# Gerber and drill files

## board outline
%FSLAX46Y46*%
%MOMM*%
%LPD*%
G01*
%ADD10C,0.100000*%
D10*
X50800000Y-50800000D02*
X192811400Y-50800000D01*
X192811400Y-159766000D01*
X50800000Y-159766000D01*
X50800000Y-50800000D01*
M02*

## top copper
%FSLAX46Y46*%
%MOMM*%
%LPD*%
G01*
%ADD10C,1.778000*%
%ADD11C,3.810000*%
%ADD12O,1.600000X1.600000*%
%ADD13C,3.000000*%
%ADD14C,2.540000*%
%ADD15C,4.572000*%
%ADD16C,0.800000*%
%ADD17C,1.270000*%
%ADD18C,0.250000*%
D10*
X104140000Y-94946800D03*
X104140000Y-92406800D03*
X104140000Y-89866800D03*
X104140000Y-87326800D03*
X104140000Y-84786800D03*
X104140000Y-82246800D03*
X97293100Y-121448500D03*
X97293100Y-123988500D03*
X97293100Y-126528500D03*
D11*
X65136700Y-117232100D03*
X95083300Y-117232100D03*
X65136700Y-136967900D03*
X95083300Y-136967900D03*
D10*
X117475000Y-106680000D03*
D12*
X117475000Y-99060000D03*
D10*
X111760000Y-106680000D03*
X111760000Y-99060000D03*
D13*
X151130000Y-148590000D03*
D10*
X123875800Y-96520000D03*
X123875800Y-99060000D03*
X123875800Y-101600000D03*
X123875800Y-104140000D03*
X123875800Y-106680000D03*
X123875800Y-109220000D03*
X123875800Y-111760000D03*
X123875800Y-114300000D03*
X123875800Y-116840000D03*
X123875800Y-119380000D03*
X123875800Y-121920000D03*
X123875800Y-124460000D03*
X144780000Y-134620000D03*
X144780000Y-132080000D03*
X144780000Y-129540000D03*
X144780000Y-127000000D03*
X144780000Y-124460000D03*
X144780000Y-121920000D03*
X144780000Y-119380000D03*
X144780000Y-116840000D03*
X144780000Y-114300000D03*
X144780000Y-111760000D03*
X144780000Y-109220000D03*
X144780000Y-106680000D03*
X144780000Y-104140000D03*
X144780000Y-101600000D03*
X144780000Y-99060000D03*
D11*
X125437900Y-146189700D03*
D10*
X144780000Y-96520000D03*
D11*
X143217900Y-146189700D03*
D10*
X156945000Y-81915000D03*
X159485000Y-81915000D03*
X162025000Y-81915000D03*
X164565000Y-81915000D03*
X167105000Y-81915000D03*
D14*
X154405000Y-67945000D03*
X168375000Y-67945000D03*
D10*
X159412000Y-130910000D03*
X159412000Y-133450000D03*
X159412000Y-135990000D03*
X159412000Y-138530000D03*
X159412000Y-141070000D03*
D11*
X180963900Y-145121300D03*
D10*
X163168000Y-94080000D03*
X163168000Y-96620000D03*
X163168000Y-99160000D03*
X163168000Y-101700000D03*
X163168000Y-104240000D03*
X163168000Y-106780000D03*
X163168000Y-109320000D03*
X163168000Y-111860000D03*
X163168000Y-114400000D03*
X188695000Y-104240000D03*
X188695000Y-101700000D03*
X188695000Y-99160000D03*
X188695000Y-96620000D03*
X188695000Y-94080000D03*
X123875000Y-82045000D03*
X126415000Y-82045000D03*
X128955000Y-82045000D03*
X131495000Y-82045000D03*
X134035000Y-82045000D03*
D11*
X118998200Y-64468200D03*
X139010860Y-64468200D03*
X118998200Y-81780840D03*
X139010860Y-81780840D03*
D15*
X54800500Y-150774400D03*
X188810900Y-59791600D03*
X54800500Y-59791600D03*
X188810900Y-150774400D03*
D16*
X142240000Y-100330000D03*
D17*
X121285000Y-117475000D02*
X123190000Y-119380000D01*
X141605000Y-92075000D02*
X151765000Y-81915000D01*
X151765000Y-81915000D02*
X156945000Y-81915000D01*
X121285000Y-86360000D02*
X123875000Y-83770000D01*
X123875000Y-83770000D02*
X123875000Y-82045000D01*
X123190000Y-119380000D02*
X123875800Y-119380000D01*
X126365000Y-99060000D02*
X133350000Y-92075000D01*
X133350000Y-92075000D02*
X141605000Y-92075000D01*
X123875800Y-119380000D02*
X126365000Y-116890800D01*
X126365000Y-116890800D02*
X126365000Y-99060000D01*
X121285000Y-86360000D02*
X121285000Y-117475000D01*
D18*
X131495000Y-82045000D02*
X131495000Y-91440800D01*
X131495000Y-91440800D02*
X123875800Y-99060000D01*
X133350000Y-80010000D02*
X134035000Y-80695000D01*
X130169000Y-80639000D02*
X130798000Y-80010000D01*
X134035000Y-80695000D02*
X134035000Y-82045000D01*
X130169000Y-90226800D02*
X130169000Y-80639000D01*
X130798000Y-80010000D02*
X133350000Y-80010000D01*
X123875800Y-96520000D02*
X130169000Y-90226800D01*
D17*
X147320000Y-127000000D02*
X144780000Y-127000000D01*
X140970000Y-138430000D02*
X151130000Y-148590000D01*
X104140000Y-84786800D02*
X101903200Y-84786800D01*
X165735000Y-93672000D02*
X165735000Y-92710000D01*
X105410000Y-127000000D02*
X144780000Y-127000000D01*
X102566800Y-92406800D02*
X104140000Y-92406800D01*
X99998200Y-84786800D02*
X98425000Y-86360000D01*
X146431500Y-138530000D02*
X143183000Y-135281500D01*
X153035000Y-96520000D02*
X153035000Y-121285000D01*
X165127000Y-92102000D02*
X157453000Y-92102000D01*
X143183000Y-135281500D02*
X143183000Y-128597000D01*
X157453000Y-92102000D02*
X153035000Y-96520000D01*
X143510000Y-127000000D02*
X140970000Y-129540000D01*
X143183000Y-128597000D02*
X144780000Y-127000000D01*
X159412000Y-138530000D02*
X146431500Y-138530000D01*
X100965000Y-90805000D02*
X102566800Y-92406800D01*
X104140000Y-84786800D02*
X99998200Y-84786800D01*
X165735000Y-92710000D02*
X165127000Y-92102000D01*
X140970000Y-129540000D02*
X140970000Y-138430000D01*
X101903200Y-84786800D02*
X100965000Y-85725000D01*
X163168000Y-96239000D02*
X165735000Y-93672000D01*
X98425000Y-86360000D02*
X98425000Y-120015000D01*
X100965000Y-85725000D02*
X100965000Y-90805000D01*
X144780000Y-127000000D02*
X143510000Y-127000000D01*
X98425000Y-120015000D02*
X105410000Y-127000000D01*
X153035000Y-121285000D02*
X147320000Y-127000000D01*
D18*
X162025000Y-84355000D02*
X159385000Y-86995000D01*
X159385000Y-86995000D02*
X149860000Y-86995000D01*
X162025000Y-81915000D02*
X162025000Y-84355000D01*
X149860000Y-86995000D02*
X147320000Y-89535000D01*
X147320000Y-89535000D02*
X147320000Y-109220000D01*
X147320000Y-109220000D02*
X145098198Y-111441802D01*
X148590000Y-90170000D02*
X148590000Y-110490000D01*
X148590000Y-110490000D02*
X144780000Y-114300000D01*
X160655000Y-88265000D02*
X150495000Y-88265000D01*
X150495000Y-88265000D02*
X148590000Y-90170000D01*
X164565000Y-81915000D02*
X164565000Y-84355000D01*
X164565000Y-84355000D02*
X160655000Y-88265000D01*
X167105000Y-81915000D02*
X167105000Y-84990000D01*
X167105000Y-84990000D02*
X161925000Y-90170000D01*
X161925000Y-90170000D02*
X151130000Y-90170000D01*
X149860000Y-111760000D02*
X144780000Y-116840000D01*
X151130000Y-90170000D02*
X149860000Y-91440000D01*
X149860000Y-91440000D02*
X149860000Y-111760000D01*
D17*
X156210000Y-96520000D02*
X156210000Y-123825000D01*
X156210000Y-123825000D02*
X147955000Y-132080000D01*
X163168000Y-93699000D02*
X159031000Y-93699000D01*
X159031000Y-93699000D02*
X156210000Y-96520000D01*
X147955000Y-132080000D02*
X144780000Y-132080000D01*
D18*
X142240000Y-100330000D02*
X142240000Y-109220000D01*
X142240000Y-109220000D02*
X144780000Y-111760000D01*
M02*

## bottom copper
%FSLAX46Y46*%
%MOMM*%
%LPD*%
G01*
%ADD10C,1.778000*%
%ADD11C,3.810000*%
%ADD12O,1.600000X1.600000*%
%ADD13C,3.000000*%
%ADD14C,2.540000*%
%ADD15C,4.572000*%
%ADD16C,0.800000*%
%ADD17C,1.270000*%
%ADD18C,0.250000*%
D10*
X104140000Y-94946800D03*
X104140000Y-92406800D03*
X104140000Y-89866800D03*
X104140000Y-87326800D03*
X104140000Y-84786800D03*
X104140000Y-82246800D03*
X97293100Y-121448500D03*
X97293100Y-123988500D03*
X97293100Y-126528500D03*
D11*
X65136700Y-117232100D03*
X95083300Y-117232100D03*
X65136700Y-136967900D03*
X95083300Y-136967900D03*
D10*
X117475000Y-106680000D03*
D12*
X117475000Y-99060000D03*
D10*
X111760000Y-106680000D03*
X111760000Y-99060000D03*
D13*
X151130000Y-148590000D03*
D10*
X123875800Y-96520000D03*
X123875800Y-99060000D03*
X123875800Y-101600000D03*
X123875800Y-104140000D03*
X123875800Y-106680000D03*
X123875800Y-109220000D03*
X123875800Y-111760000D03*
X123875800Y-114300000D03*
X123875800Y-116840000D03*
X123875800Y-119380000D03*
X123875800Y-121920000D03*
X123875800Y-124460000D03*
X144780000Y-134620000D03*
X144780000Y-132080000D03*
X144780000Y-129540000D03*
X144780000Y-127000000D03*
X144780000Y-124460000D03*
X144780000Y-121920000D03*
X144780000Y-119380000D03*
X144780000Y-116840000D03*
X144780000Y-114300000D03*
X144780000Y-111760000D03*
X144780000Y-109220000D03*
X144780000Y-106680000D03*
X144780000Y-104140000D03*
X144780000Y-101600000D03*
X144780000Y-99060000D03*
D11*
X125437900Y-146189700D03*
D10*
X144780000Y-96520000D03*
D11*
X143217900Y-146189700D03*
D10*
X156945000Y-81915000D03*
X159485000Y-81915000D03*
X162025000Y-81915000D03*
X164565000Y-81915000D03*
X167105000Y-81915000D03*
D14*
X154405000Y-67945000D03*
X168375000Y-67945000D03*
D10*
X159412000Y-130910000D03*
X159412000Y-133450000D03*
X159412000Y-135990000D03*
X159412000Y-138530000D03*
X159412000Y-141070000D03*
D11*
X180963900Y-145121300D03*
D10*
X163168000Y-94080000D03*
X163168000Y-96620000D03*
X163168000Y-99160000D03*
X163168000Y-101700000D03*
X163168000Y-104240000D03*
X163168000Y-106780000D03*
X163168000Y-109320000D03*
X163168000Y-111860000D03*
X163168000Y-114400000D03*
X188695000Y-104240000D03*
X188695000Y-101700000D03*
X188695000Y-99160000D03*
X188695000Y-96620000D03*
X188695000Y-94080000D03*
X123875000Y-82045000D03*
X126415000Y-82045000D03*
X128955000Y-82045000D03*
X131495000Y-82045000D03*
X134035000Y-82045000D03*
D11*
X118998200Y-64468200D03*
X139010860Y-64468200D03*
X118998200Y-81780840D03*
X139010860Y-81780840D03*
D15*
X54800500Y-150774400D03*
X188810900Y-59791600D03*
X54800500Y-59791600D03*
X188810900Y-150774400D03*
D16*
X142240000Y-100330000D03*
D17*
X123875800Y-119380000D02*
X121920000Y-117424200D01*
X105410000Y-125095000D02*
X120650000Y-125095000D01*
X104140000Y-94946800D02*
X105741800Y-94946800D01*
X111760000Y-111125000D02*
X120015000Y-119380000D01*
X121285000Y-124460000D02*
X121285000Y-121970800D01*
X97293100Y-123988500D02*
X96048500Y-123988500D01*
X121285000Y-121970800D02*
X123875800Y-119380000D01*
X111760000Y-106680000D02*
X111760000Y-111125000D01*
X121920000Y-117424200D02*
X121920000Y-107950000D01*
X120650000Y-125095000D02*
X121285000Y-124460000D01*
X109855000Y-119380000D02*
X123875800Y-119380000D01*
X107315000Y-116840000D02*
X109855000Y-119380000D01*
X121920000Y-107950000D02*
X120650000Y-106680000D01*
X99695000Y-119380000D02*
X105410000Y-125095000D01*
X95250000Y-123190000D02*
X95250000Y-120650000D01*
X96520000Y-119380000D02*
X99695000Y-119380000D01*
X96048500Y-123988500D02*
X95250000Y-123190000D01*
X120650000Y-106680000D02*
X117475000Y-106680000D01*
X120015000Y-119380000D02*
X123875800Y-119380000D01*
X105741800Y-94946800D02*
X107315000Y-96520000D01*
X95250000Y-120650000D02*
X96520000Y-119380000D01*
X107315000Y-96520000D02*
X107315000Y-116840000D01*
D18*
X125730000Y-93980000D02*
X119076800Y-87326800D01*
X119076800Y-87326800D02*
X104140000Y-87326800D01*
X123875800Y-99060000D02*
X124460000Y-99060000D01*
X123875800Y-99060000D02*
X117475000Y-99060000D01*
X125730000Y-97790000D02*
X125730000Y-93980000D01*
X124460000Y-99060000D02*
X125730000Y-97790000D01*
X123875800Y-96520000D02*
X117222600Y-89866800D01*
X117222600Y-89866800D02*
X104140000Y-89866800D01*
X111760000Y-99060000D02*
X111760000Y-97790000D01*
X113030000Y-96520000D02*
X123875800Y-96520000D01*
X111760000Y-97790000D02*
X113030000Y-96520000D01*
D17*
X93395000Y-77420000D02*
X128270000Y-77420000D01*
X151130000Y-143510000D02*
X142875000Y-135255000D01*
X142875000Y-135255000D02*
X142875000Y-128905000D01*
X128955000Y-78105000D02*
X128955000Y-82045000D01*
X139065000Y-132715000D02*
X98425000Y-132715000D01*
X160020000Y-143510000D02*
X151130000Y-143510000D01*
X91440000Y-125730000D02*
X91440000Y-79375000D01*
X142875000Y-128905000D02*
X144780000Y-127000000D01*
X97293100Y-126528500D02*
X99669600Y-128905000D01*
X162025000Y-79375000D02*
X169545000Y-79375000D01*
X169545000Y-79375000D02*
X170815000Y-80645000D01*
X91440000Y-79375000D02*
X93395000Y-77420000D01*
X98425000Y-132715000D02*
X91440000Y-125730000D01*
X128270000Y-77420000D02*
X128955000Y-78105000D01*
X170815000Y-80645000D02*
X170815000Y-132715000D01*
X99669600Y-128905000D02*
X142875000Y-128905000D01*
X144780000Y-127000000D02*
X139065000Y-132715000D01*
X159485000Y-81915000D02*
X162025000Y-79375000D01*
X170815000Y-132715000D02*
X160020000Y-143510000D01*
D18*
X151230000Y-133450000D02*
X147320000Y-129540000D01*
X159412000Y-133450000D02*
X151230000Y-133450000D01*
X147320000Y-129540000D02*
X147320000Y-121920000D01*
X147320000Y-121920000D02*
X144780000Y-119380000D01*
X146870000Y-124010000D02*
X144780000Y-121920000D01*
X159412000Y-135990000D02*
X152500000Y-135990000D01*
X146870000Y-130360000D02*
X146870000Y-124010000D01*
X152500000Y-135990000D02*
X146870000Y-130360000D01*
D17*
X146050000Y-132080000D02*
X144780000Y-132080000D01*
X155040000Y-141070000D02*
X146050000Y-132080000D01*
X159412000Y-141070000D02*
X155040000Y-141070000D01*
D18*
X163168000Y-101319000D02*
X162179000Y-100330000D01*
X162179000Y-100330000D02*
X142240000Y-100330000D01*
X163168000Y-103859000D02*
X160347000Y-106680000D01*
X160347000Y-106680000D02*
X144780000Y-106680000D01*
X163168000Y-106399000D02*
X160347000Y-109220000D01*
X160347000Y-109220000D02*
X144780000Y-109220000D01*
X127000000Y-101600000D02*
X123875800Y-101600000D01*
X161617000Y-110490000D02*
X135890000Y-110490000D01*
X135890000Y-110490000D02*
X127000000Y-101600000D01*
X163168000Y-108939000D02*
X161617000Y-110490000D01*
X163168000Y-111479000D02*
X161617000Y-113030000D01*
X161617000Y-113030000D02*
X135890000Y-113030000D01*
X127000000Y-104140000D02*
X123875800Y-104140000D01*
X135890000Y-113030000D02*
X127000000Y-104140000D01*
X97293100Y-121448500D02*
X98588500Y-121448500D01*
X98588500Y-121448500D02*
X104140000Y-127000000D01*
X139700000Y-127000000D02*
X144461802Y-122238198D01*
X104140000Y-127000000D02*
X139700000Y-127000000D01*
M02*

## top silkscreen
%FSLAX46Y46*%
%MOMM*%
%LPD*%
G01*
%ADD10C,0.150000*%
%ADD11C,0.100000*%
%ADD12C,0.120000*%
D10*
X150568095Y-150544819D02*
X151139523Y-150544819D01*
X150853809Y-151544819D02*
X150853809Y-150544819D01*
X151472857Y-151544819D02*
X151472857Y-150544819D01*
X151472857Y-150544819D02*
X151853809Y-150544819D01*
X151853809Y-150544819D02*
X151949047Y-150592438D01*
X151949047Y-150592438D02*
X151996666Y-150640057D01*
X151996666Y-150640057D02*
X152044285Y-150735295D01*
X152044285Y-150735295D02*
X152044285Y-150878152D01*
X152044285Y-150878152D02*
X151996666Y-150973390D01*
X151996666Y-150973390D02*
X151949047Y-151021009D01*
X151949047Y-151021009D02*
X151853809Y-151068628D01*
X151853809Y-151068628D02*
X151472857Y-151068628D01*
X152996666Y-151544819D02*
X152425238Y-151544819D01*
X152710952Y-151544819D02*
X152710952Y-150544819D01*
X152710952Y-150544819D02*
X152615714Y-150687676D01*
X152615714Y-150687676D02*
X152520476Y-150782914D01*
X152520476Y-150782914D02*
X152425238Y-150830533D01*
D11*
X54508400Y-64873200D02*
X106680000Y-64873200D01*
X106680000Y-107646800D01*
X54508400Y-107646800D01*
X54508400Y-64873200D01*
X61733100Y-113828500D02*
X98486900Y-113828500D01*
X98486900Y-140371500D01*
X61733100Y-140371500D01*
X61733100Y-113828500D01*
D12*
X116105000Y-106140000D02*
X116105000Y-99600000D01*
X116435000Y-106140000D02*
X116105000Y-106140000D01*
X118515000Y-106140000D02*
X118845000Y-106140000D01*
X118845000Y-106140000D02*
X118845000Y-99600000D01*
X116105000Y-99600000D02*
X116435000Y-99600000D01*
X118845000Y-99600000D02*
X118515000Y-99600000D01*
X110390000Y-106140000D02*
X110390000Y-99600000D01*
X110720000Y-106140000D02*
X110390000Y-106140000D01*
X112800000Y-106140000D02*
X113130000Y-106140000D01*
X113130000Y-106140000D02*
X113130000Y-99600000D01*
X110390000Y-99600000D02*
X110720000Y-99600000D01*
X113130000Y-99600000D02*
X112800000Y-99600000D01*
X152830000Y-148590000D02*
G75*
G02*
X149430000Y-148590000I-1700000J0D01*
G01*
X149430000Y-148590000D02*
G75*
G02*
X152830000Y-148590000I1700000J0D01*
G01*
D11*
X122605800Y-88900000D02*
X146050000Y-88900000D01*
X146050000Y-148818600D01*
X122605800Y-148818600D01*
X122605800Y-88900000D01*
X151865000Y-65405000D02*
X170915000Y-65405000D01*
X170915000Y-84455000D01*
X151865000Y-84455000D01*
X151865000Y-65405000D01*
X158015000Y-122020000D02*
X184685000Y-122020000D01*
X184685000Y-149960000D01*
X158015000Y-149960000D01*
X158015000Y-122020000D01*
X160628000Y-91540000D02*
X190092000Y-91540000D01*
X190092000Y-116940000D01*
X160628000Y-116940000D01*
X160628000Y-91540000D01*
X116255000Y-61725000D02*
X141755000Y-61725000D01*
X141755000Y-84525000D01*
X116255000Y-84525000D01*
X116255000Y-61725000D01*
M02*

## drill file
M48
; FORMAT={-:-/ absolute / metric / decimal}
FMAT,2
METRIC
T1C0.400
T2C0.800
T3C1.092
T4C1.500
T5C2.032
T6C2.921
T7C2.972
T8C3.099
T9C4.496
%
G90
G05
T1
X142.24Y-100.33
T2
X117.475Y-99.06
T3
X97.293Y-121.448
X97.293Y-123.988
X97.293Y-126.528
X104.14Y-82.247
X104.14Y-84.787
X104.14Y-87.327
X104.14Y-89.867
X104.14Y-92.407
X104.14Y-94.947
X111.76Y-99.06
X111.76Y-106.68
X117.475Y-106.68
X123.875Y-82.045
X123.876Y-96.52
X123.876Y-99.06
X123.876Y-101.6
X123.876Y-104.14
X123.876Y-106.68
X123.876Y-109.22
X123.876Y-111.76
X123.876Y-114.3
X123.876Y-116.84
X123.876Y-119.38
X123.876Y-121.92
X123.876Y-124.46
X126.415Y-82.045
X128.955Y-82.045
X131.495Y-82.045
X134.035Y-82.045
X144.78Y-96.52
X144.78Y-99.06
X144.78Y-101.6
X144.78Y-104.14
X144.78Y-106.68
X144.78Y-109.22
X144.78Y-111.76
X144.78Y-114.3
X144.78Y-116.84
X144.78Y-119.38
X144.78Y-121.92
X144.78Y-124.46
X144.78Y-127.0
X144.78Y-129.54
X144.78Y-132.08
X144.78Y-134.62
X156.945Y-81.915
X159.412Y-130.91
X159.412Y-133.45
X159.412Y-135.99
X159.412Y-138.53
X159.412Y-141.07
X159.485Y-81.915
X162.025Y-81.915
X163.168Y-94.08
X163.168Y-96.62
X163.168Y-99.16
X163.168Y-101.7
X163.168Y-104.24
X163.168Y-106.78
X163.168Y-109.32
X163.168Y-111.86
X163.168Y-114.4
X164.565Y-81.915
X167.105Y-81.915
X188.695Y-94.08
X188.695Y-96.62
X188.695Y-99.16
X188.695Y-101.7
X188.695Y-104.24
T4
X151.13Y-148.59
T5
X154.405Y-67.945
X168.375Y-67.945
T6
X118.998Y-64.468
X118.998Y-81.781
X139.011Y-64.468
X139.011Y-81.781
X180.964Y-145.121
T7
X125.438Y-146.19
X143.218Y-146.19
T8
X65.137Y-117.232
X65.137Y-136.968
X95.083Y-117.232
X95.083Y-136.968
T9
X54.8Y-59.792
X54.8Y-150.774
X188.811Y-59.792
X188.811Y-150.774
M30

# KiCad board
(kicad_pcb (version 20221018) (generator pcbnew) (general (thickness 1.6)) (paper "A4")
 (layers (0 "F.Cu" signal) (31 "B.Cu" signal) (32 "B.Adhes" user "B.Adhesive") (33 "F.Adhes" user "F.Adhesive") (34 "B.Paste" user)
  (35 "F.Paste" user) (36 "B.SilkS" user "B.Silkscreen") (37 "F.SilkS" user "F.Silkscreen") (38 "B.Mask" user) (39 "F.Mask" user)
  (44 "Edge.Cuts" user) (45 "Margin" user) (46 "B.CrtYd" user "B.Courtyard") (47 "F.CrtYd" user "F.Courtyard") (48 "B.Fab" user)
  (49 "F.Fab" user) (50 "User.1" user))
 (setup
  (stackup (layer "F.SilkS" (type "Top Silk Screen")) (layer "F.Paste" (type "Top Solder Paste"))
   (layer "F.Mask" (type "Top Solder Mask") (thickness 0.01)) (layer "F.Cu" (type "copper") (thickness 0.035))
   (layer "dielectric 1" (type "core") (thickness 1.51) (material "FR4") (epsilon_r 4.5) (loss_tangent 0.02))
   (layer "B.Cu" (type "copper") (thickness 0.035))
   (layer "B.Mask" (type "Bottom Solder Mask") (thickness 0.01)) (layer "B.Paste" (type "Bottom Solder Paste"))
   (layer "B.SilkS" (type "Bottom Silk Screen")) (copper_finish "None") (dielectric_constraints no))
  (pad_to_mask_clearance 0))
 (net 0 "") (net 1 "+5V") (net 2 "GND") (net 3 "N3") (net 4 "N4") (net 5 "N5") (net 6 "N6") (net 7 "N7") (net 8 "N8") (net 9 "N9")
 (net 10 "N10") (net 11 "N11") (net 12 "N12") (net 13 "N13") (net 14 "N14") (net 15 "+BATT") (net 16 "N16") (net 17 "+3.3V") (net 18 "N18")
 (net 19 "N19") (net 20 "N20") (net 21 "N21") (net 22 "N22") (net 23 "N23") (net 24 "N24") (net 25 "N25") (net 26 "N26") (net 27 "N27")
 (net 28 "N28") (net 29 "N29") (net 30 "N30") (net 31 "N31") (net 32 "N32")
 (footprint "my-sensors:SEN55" (layer "F.Cu") (at 106.68 107.6468 180)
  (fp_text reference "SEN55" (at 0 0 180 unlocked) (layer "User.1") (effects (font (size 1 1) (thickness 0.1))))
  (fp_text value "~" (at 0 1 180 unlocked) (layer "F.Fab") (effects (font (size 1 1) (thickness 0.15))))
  (fp_rect (start 0 0) (end 52.1716 42.7736) (stroke (width 0.1) (type default)) (fill none) (layer "F.SilkS"))
  (pad "1" thru_hole circle (at 2.54 12.7 180) (size 1.778 1.778) (drill 1.0922) (layers "*.Cu" "*.Mask") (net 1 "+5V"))
  (pad "2" thru_hole circle (at 2.54 15.24 180) (size 1.778 1.778) (drill 1.0922) (layers "*.Cu" "*.Mask") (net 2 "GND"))
  (pad "3" thru_hole circle (at 2.54 17.78 180) (size 1.778 1.778) (drill 1.0922) (layers "*.Cu" "*.Mask") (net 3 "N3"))
  (pad "4" thru_hole circle (at 2.54 20.32 180) (size 1.778 1.778) (drill 1.0922) (layers "*.Cu" "*.Mask") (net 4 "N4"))
  (pad "5" thru_hole circle (at 2.54 22.86 180) (size 1.778 1.778) (drill 1.0922) (layers "*.Cu" "*.Mask") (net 2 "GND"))
  (pad "6" thru_hole circle (at 2.54 25.4 180) (size 1.778 1.778) (drill 1.0922) (layers "*.Cu" "*.Mask") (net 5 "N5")))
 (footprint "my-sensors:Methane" (layer "F.Cu") (at 61.7331 113.8285)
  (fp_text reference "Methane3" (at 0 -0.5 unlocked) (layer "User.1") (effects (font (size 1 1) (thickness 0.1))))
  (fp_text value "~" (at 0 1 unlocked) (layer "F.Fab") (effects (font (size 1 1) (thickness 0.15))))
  (fp_rect (start 0 0) (end 36.7538 26.543) (stroke (width 0.1) (type default)) (fill none) (layer "F.SilkS"))
  (pad "1" thru_hole circle (at 35.56 7.62) (size 1.778 1.778) (drill 1.0922) (layers "*.Cu" "*.Mask") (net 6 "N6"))
  (pad "2" thru_hole circle (at 35.56 10.16) (size 1.778 1.778) (drill 1.0922) (layers "*.Cu" "*.Mask") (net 1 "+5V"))
  (pad "3" thru_hole circle (at 35.56 12.7) (size 1.778 1.778) (drill 1.0922) (layers "*.Cu" "*.Mask") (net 2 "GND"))
  (pad "4" thru_hole circle (at 3.4036 3.4036 270) (size 3.81 3.81) (drill 3.0988) (layers "*.Cu" "*.Mask"))
  (pad "5" thru_hole circle (at 33.3502 3.4036 270) (size 3.81 3.81) (drill 3.0988) (layers "*.Cu" "*.Mask"))
  (pad "6" thru_hole circle (at 3.4036 23.1394 270) (size 3.81 3.81) (drill 3.0988) (layers "*.Cu" "*.Mask"))
  (pad "7" thru_hole circle (at 33.3502 23.1394 270) (size 3.81 3.81) (drill 3.0988) (layers "*.Cu" "*.Mask")))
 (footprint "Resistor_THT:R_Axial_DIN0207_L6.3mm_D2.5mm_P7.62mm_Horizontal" (layer "F.Cu") (at 117.475 106.68 90)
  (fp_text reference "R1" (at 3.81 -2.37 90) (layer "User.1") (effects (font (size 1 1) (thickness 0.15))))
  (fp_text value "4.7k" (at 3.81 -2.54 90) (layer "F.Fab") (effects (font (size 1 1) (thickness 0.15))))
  (fp_line (start 0.54 -1.37) (end 7.08 -1.37) (stroke (width 0.12) (type solid)) (layer "F.SilkS"))
  (fp_line (start 0.54 -1.04) (end 0.54 -1.37) (stroke (width 0.12) (type solid)) (layer "F.SilkS"))
  (fp_line (start 0.54 1.04) (end 0.54 1.37) (stroke (width 0.12) (type solid)) (layer "F.SilkS"))
  (fp_line (start 0.54 1.37) (end 7.08 1.37) (stroke (width 0.12) (type solid)) (layer "F.SilkS"))
  (fp_line (start 7.08 -1.37) (end 7.08 -1.04) (stroke (width 0.12) (type solid)) (layer "F.SilkS"))
  (fp_line (start 7.08 1.37) (end 7.08 1.04) (stroke (width 0.12) (type solid)) (layer "F.SilkS"))
  (pad "1" thru_hole circle (at 0 0 90) (size 1.778 1.778) (drill 1.0922) (layers "*.Cu" "*.Mask") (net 1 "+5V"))
  (pad "2" thru_hole oval (at 7.62 0 90) (size 1.6 1.6) (drill 0.8) (layers "*.Cu" "*.Mask") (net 4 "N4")))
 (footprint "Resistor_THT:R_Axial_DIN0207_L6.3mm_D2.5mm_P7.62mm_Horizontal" (layer "F.Cu") (at 111.76 106.68 90)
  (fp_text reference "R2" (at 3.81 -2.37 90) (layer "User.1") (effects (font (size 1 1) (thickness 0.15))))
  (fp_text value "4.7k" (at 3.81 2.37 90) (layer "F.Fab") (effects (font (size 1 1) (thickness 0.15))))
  (fp_line (start 0.54 -1.37) (end 7.08 -1.37) (stroke (width 0.12) (type solid)) (layer "F.SilkS"))
  (fp_line (start 0.54 -1.04) (end 0.54 -1.37) (stroke (width 0.12) (type solid)) (layer "F.SilkS"))
  (fp_line (start 0.54 1.04) (end 0.54 1.37) (stroke (width 0.12) (type solid)) (layer "F.SilkS"))
  (fp_line (start 0.54 1.37) (end 7.08 1.37) (stroke (width 0.12) (type solid)) (layer "F.SilkS"))
  (fp_line (start 7.08 -1.37) (end 7.08 -1.04) (stroke (width 0.12) (type solid)) (layer "F.SilkS"))
  (fp_line (start 7.08 1.37) (end 7.08 1.04) (stroke (width 0.12) (type solid)) (layer "F.SilkS"))
  (pad "1" thru_hole circle (at 0 0 90) (size 1.778 1.778) (drill 1.0922) (layers "*.Cu" "*.Mask") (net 1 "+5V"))
  (pad "2" thru_hole circle (at 7.62 0 90) (size 1.778 1.778) (drill 1.0922) (layers "*.Cu" "*.Mask") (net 3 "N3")))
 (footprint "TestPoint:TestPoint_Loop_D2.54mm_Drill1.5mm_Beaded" (layer "F.Cu") (at 151.13 148.59)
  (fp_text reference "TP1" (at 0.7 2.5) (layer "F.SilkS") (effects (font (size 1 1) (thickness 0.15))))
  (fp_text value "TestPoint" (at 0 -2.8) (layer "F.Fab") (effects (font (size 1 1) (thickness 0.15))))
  (fp_circle (center 0 0) (end 1.7 0) (stroke (width 0.12) (type solid)) (fill none) (layer "F.SilkS"))
  (pad "1" thru_hole circle (at 0 0) (size 3 3) (drill 1.5) (layers "*.Cu" "*.Mask") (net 2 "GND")))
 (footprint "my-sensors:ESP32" (layer "F.Cu") (at 122.6058 88.9)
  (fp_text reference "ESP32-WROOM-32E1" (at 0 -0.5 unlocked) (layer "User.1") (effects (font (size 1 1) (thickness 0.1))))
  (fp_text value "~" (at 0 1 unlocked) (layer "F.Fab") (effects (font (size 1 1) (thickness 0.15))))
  (fp_rect (start 0 0) (end 23.4442 59.9186) (stroke (width 0.1) (type default)) (fill none) (layer "F.SilkS"))
  (pad "1" thru_hole circle (at 1.27 7.62) (size 1.778 1.778) (drill 1.0922) (layers "*.Cu" "*.Mask") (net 3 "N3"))
  (pad "2" thru_hole circle (at 1.27 10.16) (size 1.778 1.778) (drill 1.0922) (layers "*.Cu" "*.Mask") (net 4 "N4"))
  (pad "3" thru_hole circle (at 1.27 12.7) (size 1.778 1.778) (drill 1.0922) (layers "*.Cu" "*.Mask") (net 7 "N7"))
  (pad "4" thru_hole circle (at 1.27 15.24) (size 1.778 1.778) (drill 1.0922) (layers "*.Cu" "*.Mask") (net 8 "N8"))
  (pad "5" thru_hole circle (at 1.27 17.78) (size 1.778 1.778) (drill 1.0922) (layers "*.Cu" "*.Mask") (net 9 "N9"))
  (pad "6" thru_hole circle (at 1.27 20.32) (size 1.778 1.778) (drill 1.0922) (layers "*.Cu" "*.Mask") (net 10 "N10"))
  (pad "7" thru_hole circle (at 1.27 22.86) (size 1.778 1.778) (drill 1.0922) (layers "*.Cu" "*.Mask") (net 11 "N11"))
  (pad "8" thru_hole circle (at 1.27 25.4) (size 1.778 1.778) (drill 1.0922) (layers "*.Cu" "*.Mask") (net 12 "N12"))
  (pad "9" thru_hole circle (at 1.27 27.94) (size 1.778 1.778) (drill 1.0922) (layers "*.Cu" "*.Mask") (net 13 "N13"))
  (pad "10" thru_hole circle (at 1.27 30.48) (size 1.778 1.778) (drill 1.0922) (layers "*.Cu" "*.Mask") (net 1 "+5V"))
  (pad "11" thru_hole circle (at 1.27 33.02) (size 1.778 1.778) (drill 1.0922) (layers "*.Cu" "*.Mask") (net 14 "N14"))
  (pad "12" thru_hole circle (at 1.27 35.56) (size 1.778 1.778) (drill 1.0922) (layers "*.Cu" "*.Mask") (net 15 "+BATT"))
  (pad "13" thru_hole circle (at 22.1742 45.72) (size 1.778 1.778) (drill 1.0922) (layers "*.Cu" "*.Mask") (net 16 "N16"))
  (pad "14" thru_hole circle (at 22.1742 43.18) (size 1.778 1.778) (drill 1.0922) (layers "*.Cu" "*.Mask") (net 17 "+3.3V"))
  (pad "15" thru_hole circle (at 22.1742 40.64) (size 1.778 1.778) (drill 1.0922) (layers "*.Cu" "*.Mask") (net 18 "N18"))
  (pad "16" thru_hole circle (at 22.1742 38.1) (size 1.778 1.778) (drill 1.0922) (layers "*.Cu" "*.Mask") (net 2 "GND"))
  (pad "17" thru_hole circle (at 22.1742 35.56) (size 1.778 1.778) (drill 1.0922) (layers "*.Cu" "*.Mask") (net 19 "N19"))
  (pad "18" thru_hole circle (at 22.1742 33.02) (size 1.778 1.778) (drill 1.0922) (layers "*.Cu" "*.Mask") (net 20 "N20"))
  (pad "19" thru_hole circle (at 22.1742 30.48) (size 1.778 1.778) (drill 1.0922) (layers "*.Cu" "*.Mask") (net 6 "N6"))
  (pad "20" thru_hole circle (at 22.1742 27.94) (size 1.778 1.778) (drill 1.0922) (layers "*.Cu" "*.Mask") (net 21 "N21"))
  (pad "21" thru_hole circle (at 22.1742 25.4) (size 1.778 1.778) (drill 1.0922) (layers "*.Cu" "*.Mask") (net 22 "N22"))
  (pad "22" thru_hole circle (at 22.1742 22.86) (size 1.778 1.778) (drill 1.0922) (layers "*.Cu" "*.Mask") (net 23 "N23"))
  (pad "23" thru_hole circle (at 22.1742 20.32) (size 1.778 1.778) (drill 1.0922) (layers "*.Cu" "*.Mask") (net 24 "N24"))
  (pad "24" thru_hole circle (at 22.1742 17.78) (size 1.778 1.778) (drill 1.0922) (layers "*.Cu" "*.Mask") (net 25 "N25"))
  (pad "25" thru_hole circle (at 22.1742 15.24) (size 1.778 1.778) (drill 1.0922) (layers "*.Cu" "*.Mask") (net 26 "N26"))
  (pad "26" thru_hole circle (at 22.1742 12.7) (size 1.778 1.778) (drill 1.0922) (layers "*.Cu" "*.Mask") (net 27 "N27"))
  (pad "27" thru_hole circle (at 22.1742 10.16) (size 1.778 1.778) (drill 1.0922) (layers "*.Cu" "*.Mask") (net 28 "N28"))
  (pad "28" thru_hole circle (at 2.8321 57.2897) (size 3.81 3.81) (drill 2.9718) (layers "*.Cu" "*.Mask") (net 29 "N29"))
  (pad "28" thru_hole circle (at 22.1742 7.62) (size 1.778 1.778) (drill 1.0922) (layers "*.Cu" "*.Mask") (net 29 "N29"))
  (pad "29" thru_hole circle (at 20.6121 57.2897) (size 3.81 3.81) (drill 2.9718) (layers "*.Cu" "*.Mask")))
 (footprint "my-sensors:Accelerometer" (layer "F.Cu") (at 151.865 65.405)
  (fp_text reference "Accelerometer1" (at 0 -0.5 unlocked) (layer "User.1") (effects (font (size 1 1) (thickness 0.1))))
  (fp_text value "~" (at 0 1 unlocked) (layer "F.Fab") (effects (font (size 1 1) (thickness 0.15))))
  (fp_rect (start 0 0) (end 19.05 19.05) (stroke (width 0.1) (type default)) (fill none) (layer "F.SilkS"))
  (pad "1" thru_hole circle (at 5.08 16.51) (size 1.778 1.778) (drill 1.0922) (layers "*.Cu" "*.Mask") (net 1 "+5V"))
  (pad "2" thru_hole circle (at 7.62 16.51) (size 1.778 1.778) (drill 1.0922) (layers "*.Cu" "*.Mask") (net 2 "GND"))
  (pad "3" thru_hole circle (at 10.16 16.51) (size 1.778 1.778) (drill 1.0922) (layers "*.Cu" "*.Mask") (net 23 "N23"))
  (pad "4" thru_hole circle (at 12.7 16.51) (size 1.778 1.778) (drill 1.0922) (layers "*.Cu" "*.Mask") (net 22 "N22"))
  (pad "5" thru_hole circle (at 15.24 16.51) (size 1.778 1.778) (drill 1.0922) (layers "*.Cu" "*.Mask") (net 21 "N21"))
  (pad "6" thru_hole circle (at 2.54 2.54) (size 2.54 2.54) (drill 2.032) (layers "*.Cu" "*.Mask"))
  (pad "7" thru_hole circle (at 16.51 2.54) (size 2.54 2.54) (drill 2.032) (layers "*.Cu" "*.Mask")))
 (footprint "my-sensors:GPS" (layer "F.Cu") (at 184.685 122.02 -90)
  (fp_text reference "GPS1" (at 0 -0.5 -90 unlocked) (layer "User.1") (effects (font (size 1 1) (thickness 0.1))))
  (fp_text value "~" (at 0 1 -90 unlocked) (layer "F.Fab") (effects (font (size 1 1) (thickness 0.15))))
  (fp_rect (start 0 0) (end 27.94 26.67) (stroke (width 0.1) (type default)) (fill none) (layer "F.SilkS"))
  (pad "1" thru_hole circle (at 8.89 25.273 270) (size 1.778 1.778) (drill 1.0922) (layers "*.Cu" "*.Mask") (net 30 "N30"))
  (pad "2" thru_hole circle (at 11.43 25.273 270) (size 1.778 1.778) (drill 1.0922) (layers "*.Cu" "*.Mask") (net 28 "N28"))
  (pad "3" thru_hole circle (at 13.97 25.273 270) (size 1.778 1.778) (drill 1.0922) (layers "*.Cu" "*.Mask") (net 27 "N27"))
  (pad "4" thru_hole circle (at 16.51 25.273 270) (size 1.778 1.778) (drill 1.0922) (layers "*.Cu" "*.Mask") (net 2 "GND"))
  (pad "5" thru_hole circle (at 19.05 25.273 270) (size 1.778 1.778) (drill 1.0922) (layers "*.Cu" "*.Mask") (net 17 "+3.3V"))
  (pad "6" thru_hole circle (at 23.1013 3.7211 270) (size 3.81 3.81) (drill 2.921) (layers "*.Cu" "*.Mask")))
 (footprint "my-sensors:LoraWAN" (layer "F.Cu") (at 160.628 91.54)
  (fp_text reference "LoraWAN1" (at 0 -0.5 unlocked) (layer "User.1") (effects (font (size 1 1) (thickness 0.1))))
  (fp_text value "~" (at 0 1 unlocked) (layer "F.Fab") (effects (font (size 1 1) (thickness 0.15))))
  (fp_rect (start 0 0) (end 29.464 25.4) (stroke (width 0.1) (type default)) (fill none) (layer "F.SilkS"))
  (pad "1" thru_hole circle (at 2.54 2.54 270) (size 1.778 1.778) (drill 1.0922) (layers "*.Cu" "*.Mask") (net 17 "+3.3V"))
  (pad "2" thru_hole circle (at 2.54 5.08 270) (size 1.778 1.778) (drill 1.0922) (layers "*.Cu" "*.Mask") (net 2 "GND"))
  (pad "3" thru_hole circle (at 2.54 7.62 270) (size 1.778 1.778) (drill 1.0922) (layers "*.Cu" "*.Mask") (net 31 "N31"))
  (pad "4" thru_hole circle (at 2.54 10.16 270) (size 1.778 1.778) (drill 1.0922) (layers "*.Cu" "*.Mask") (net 24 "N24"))
  (pad "5" thru_hole circle (at 2.54 12.7 270) (size 1.778 1.778) (drill 1.0922) (layers "*.Cu" "*.Mask") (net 26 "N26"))
  (pad "6" thru_hole circle (at 2.54 15.24 270) (size 1.778 1.778) (drill 1.0922) (layers "*.Cu" "*.Mask") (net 25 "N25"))
  (pad "7" thru_hole circle (at 2.54 17.78 270) (size 1.778 1.778) (drill 1.0922) (layers "*.Cu" "*.Mask") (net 7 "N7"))
  (pad "8" thru_hole circle (at 2.54 20.32 270) (size 1.778 1.778) (drill 1.0922) (layers "*.Cu" "*.Mask") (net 8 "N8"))
  (pad "9" thru_hole circle (at 2.54 22.86 270) (size 1.778 1.778) (drill 1.0922) (layers "*.Cu" "*.Mask"))
  (pad "10" thru_hole circle (at 28.067 12.7 270) (size 1.778 1.778) (drill 1.0922) (layers "*.Cu" "*.Mask"))
  (pad "11" thru_hole circle (at 28.067 10.16 270) (size 1.778 1.778) (drill 1.0922) (layers "*.Cu" "*.Mask"))
  (pad "12" thru_hole circle (at 28.067 7.62 270) (size 1.778 1.778) (drill 1.0922) (layers "*.Cu" "*.Mask"))
  (pad "13" thru_hole circle (at 28.067 5.08 270) (size 1.778 1.778) (drill 1.0922) (layers "*.Cu" "*.Mask"))
  (pad "14" thru_hole circle (at 28.067 2.54 270) (size 1.778 1.778) (drill 1.0922) (layers "*.Cu" "*.Mask")))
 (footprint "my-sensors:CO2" (layer "F.Cu") (at 116.255 61.725)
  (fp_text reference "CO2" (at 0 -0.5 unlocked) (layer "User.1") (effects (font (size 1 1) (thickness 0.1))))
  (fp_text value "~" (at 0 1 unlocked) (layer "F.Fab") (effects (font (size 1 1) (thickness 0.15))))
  (fp_rect (start 0 0) (end 25.5 22.8) (stroke (width 0.1) (type default)) (fill none) (layer "F.SilkS"))
  (pad "1" thru_hole circle (at 7.62 20.32) (size 1.778 1.778) (drill 1.0922) (layers "*.Cu" "*.Mask") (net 1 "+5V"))
  (pad "2" thru_hole circle (at 10.16 20.32) (size 1.778 1.778) (drill 1.0922) (layers "*.Cu" "*.Mask") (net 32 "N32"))
  (pad "3" thru_hole circle (at 12.7 20.32) (size 1.778 1.778) (drill 1.0922) (layers "*.Cu" "*.Mask") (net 2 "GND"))
  (pad "4" thru_hole circle (at 15.24 20.32) (size 1.778 1.778) (drill 1.0922) (layers "*.Cu" "*.Mask") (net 4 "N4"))
  (pad "5" thru_hole circle (at 17.78 20.32) (size 1.778 1.778) (drill 1.0922) (layers "*.Cu" "*.Mask") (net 3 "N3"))
  (pad "6" thru_hole circle (at 2.7432 2.7432 270) (size 3.81 3.81) (drill 2.921) (layers "*.Cu" "*.Mask"))
  (pad "7" thru_hole circle (at 22.75586 2.7432 270) (size 3.81 3.81) (drill 2.921) (layers "*.Cu" "*.Mask"))
  (pad "8" thru_hole circle (at 2.7432 20.05584 270) (size 3.81 3.81) (drill 2.921) (layers "*.Cu" "*.Mask"))
  (pad "9" thru_hole circle (at 22.75586 20.05584 270) (size 3.81 3.81) (drill 2.921) (layers "*.Cu" "*.Mask")))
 (gr_rect (start 50.8 50.8) (end 192.8114 159.766) (stroke (width 0.1) (type default)) (fill none) (layer "Edge.Cuts"))
 (via (at 54.8005 150.7744) (size 4.572) (drill 4.4958) (layers "F.Cu" "B.Cu") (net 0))
 (via (at 188.8109 59.7916) (size 4.572) (drill 4.4958) (layers "F.Cu" "B.Cu") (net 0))
 (via (at 54.8005 59.7916) (size 4.572) (drill 4.4958) (layers "F.Cu" "B.Cu") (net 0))
 (via (at 188.8109 150.7744) (size 4.572) (drill 4.4958) (layers "F.Cu" "B.Cu") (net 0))
 (segment (start 121.285 117.475) (end 123.19 119.38) (width 1.27) (layer "F.Cu") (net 1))
 (segment (start 141.605 92.075) (end 151.765 81.915) (width 1.27) (layer "F.Cu") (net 1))
 (segment (start 151.765 81.915) (end 156.945 81.915) (width 1.27) (layer "F.Cu") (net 1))
 (segment (start 121.285 86.36) (end 123.875 83.77) (width 1.27) (layer "F.Cu") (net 1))
 (segment (start 123.875 83.77) (end 123.875 82.045) (width 1.27) (layer "F.Cu") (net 1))
 (segment (start 123.19 119.38) (end 123.8758 119.38) (width 1.27) (layer "F.Cu") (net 1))
 (segment (start 126.365 99.06) (end 133.35 92.075) (width 1.27) (layer "F.Cu") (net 1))
 (segment (start 133.35 92.075) (end 141.605 92.075) (width 1.27) (layer "F.Cu") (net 1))
 (segment (start 123.8758 119.38) (end 126.365 116.8908) (width 1.27) (layer "F.Cu") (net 1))
 (segment (start 126.365 116.8908) (end 126.365 99.06) (width 1.27) (layer "F.Cu") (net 1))
 (segment (start 121.285 86.36) (end 121.285 117.475) (width 1.27) (layer "F.Cu") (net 1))
 (segment (start 123.8758 119.38) (end 121.92 117.4242) (width 1.27) (layer "B.Cu") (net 1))
 (segment (start 105.41 125.095) (end 120.65 125.095) (width 1.27) (layer "B.Cu") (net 1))
 (segment (start 104.14 94.9468) (end 105.7418 94.9468) (width 1.27) (layer "B.Cu") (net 1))
 (segment (start 111.76 111.125) (end 120.015 119.38) (width 1.27) (layer "B.Cu") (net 1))
 (segment (start 121.285 124.46) (end 121.285 121.9708) (width 1.27) (layer "B.Cu") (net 1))
 (segment (start 97.2931 123.9885) (end 96.0485 123.9885) (width 1.27) (layer "B.Cu") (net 1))
 (segment (start 121.285 121.9708) (end 123.8758 119.38) (width 1.27) (layer "B.Cu") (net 1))
 (segment (start 111.76 106.68) (end 111.76 111.125) (width 1.27) (layer "B.Cu") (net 1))
 (segment (start 121.92 117.4242) (end 121.92 107.95) (width 1.27) (layer "B.Cu") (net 1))
 (segment (start 120.65 125.095) (end 121.285 124.46) (width 1.27) (layer "B.Cu") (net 1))
 (segment (start 109.855 119.38) (end 123.8758 119.38) (width 1.27) (layer "B.Cu") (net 1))
 (segment (start 107.315 116.84) (end 109.855 119.38) (width 1.27) (layer "B.Cu") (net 1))
 (segment (start 121.92 107.95) (end 120.65 106.68) (width 1.27) (layer "B.Cu") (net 1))
 (segment (start 99.695 119.38) (end 105.41 125.095) (width 1.27) (layer "B.Cu") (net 1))
 (segment (start 95.25 123.19) (end 95.25 120.65) (width 1.27) (layer "B.Cu") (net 1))
 (segment (start 96.52 119.38) (end 99.695 119.38) (width 1.27) (layer "B.Cu") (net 1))
 (segment (start 96.0485 123.9885) (end 95.25 123.19) (width 1.27) (layer "B.Cu") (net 1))
 (segment (start 120.65 106.68) (end 117.475 106.68) (width 1.27) (layer "B.Cu") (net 1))
 (segment (start 120.015 119.38) (end 123.8758 119.38) (width 1.27) (layer "B.Cu") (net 1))
 (segment (start 105.7418 94.9468) (end 107.315 96.52) (width 1.27) (layer "B.Cu") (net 1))
 (segment (start 95.25 120.65) (end 96.52 119.38) (width 1.27) (layer "B.Cu") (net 1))
 (segment (start 107.315 96.52) (end 107.315 116.84) (width 1.27) (layer "B.Cu") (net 1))
 (segment (start 131.495 82.045) (end 131.495 91.4408) (width 0.25) (layer "F.Cu") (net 4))
 (segment (start 131.495 91.4408) (end 123.8758 99.06) (width 0.25) (layer "F.Cu") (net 4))
 (segment (start 125.73 93.98) (end 119.0768 87.3268) (width 0.25) (layer "B.Cu") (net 4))
 (segment (start 119.0768 87.3268) (end 104.14 87.3268) (width 0.25) (layer "B.Cu") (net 4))
 (segment (start 123.8758 99.06) (end 124.46 99.06) (width 0.25) (layer "B.Cu") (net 4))
 (segment (start 123.8758 99.06) (end 117.475 99.06) (width 0.25) (layer "B.Cu") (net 4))
 (segment (start 125.73 97.79) (end 125.73 93.98) (width 0.25) (layer "B.Cu") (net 4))
 (segment (start 124.46 99.06) (end 125.73 97.79) (width 0.25) (layer "B.Cu") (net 4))
 (segment (start 133.35 80.01) (end 134.035 80.695) (width 0.25) (layer "F.Cu") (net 3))
 (segment (start 130.169 80.639) (end 130.798 80.01) (width 0.25) (layer "F.Cu") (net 3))
 (segment (start 134.035 80.695) (end 134.035 82.045) (width 0.25) (layer "F.Cu") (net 3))
 (segment (start 130.169 90.2268) (end 130.169 80.639) (width 0.25) (layer "F.Cu") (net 3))
 (segment (start 130.798 80.01) (end 133.35 80.01) (width 0.25) (layer "F.Cu") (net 3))
 (segment (start 123.8758 96.52) (end 130.169 90.2268) (width 0.25) (layer "F.Cu") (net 3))
 (segment (start 123.8758 96.52) (end 117.2226 89.8668) (width 0.25) (layer "B.Cu") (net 3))
 (segment (start 117.2226 89.8668) (end 104.14 89.8668) (width 0.25) (layer "B.Cu") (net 3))
 (segment (start 111.76 99.06) (end 111.76 97.79) (width 0.25) (layer "B.Cu") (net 3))
 (segment (start 113.03 96.52) (end 123.8758 96.52) (width 0.25) (layer "B.Cu") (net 3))
 (segment (start 111.76 97.79) (end 113.03 96.52) (width 0.25) (layer "B.Cu") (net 3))
 (segment (start 147.32 127) (end 144.78 127) (width 1.27) (layer "F.Cu") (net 2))
 (segment (start 140.97 138.43) (end 151.13 148.59) (width 1.27) (layer "F.Cu") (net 2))
 (segment (start 104.14 84.7868) (end 101.9032 84.7868) (width 1.27) (layer "F.Cu") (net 2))
 (segment (start 165.735 93.672) (end 165.735 92.71) (width 1.27) (layer "F.Cu") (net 2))
 (segment (start 105.41 127) (end 144.78 127) (width 1.27) (layer "F.Cu") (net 2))
 (segment (start 102.5668 92.4068) (end 104.14 92.4068) (width 1.27) (layer "F.Cu") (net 2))
 (segment (start 99.9982 84.7868) (end 98.425 86.36) (width 1.27) (layer "F.Cu") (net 2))
 (segment (start 146.4315 138.53) (end 143.183 135.2815) (width 1.27) (layer "F.Cu") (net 2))
 (segment (start 153.035 96.52) (end 153.035 121.285) (width 1.27) (layer "F.Cu") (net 2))
 (segment (start 165.127 92.102) (end 157.453 92.102) (width 1.27) (layer "F.Cu") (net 2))
 (segment (start 143.183 135.2815) (end 143.183 128.597) (width 1.27) (layer "F.Cu") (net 2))
 (segment (start 157.453 92.102) (end 153.035 96.52) (width 1.27) (layer "F.Cu") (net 2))
 (segment (start 143.51 127) (end 140.97 129.54) (width 1.27) (layer "F.Cu") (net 2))
 (segment (start 143.183 128.597) (end 144.78 127) (width 1.27) (layer "F.Cu") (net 2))
 (segment (start 159.412 138.53) (end 146.4315 138.53) (width 1.27) (layer "F.Cu") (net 2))
 (segment (start 100.965 90.805) (end 102.5668 92.4068) (width 1.27) (layer "F.Cu") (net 2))
 (segment (start 104.14 84.7868) (end 99.9982 84.7868) (width 1.27) (layer "F.Cu") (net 2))
 (segment (start 165.735 92.71) (end 165.127 92.102) (width 1.27) (layer "F.Cu") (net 2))
 (segment (start 140.97 129.54) (end 140.97 138.43) (width 1.27) (layer "F.Cu") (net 2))
 (segment (start 101.9032 84.7868) (end 100.965 85.725) (width 1.27) (layer "F.Cu") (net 2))
 (segment (start 163.168 96.239) (end 165.735 93.672) (width 1.27) (layer "F.Cu") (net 2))
 (segment (start 98.425 86.36) (end 98.425 120.015) (width 1.27) (layer "F.Cu") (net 2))
 (segment (start 100.965 85.725) (end 100.965 90.805) (width 1.27) (layer "F.Cu") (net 2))
 (segment (start 144.78 127) (end 143.51 127) (width 1.27) (layer "F.Cu") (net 2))
 (segment (start 98.425 120.015) (end 105.41 127) (width 1.27) (layer "F.Cu") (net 2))
 (segment (start 153.035 121.285) (end 147.32 127) (width 1.27) (layer "F.Cu") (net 2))
 (segment (start 93.395 77.42) (end 128.27 77.42) (width 1.27) (layer "B.Cu") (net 2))
 (segment (start 151.13 143.51) (end 142.875 135.255) (width 1.27) (layer "B.Cu") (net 2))
 (segment (start 142.875 135.255) (end 142.875 128.905) (width 1.27) (layer "B.Cu") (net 2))
 (segment (start 128.955 78.105) (end 128.955 82.045) (width 1.27) (layer "B.Cu") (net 2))
 (segment (start 139.065 132.715) (end 98.425 132.715) (width 1.27) (layer "B.Cu") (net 2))
 (segment (start 160.02 143.51) (end 151.13 143.51) (width 1.27) (layer "B.Cu") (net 2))
 (segment (start 91.44 125.73) (end 91.44 79.375) (width 1.27) (layer "B.Cu") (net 2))
 (segment (start 142.875 128.905) (end 144.78 127) (width 1.27) (layer "B.Cu") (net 2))
 (segment (start 97.2931 126.5285) (end 99.6696 128.905) (width 1.27) (layer "B.Cu") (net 2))
 (segment (start 162.025 79.375) (end 169.545 79.375) (width 1.27) (layer "B.Cu") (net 2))
 (segment (start 169.545 79.375) (end 170.815 80.645) (width 1.27) (layer "B.Cu") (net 2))
 (segment (start 91.44 79.375) (end 93.395 77.42) (width 1.27) (layer "B.Cu") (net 2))
 (segment (start 98.425 132.715) (end 91.44 125.73) (width 1.27) (layer "B.Cu") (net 2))
 (segment (start 128.27 77.42) (end 128.955 78.105) (width 1.27) (layer "B.Cu") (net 2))
 (segment (start 170.815 80.645) (end 170.815 132.715) (width 1.27) (layer "B.Cu") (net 2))
 (segment (start 99.6696 128.905) (end 142.875 128.905) (width 1.27) (layer "B.Cu") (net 2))
 (segment (start 144.78 127) (end 139.065 132.715) (width 1.27) (layer "B.Cu") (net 2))
 (segment (start 159.485 81.915) (end 162.025 79.375) (width 1.27) (layer "B.Cu") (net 2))
 (segment (start 170.815 132.715) (end 160.02 143.51) (width 1.27) (layer "B.Cu") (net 2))
 (segment (start 162.025 84.355) (end 159.385 86.995) (width 0.25) (layer "F.Cu") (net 23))
 (segment (start 159.385 86.995) (end 149.86 86.995) (width 0.25) (layer "F.Cu") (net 23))
 (segment (start 162.025 81.915) (end 162.025 84.355) (width 0.25) (layer "F.Cu") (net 23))
 (segment (start 149.86 86.995) (end 147.32 89.535) (width 0.25) (layer "F.Cu") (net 23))
 (segment (start 147.32 89.535) (end 147.32 109.22) (width 0.25) (layer "F.Cu") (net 23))
 (segment (start 147.32 109.22) (end 145.098198 111.441802) (width 0.25) (layer "F.Cu") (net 23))
 (segment (start 148.59 90.17) (end 148.59 110.49) (width 0.25) (layer "F.Cu") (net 22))
 (segment (start 148.59 110.49) (end 144.78 114.3) (width 0.25) (layer "F.Cu") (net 22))
 (segment (start 160.655 88.265) (end 150.495 88.265) (width 0.25) (layer "F.Cu") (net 22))
 (segment (start 150.495 88.265) (end 148.59 90.17) (width 0.25) (layer "F.Cu") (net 22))
 (segment (start 164.565 81.915) (end 164.565 84.355) (width 0.25) (layer "F.Cu") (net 22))
 (segment (start 164.565 84.355) (end 160.655 88.265) (width 0.25) (layer "F.Cu") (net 22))
 (segment (start 167.105 81.915) (end 167.105 84.99) (width 0.25) (layer "F.Cu") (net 21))
 (segment (start 167.105 84.99) (end 161.925 90.17) (width 0.25) (layer "F.Cu") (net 21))
 (segment (start 161.925 90.17) (end 151.13 90.17) (width 0.25) (layer "F.Cu") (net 21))
 (segment (start 149.86 111.76) (end 144.78 116.84) (width 0.25) (layer "F.Cu") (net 21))
 (segment (start 151.13 90.17) (end 149.86 91.44) (width 0.25) (layer "F.Cu") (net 21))
 (segment (start 149.86 91.44) (end 149.86 111.76) (width 0.25) (layer "F.Cu") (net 21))
 (segment (start 151.23 133.45) (end 147.32 129.54) (width 0.25) (layer "B.Cu") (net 28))
 (segment (start 159.412 133.45) (end 151.23 133.45) (width 0.25) (layer "B.Cu") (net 28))
 (segment (start 147.32 129.54) (end 147.32 121.92) (width 0.25) (layer "B.Cu") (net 28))
 (segment (start 147.32 121.92) (end 144.78 119.38) (width 0.25) (layer "B.Cu") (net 28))
 (segment (start 146.87 124.01) (end 144.78 121.92) (width 0.25) (layer "B.Cu") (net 27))
 (segment (start 159.412 135.99) (end 152.5 135.99) (width 0.25) (layer "B.Cu") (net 27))
 (segment (start 146.87 130.36) (end 146.87 124.01) (width 0.25) (layer "B.Cu") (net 27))
 (segment (start 152.5 135.99) (end 146.87 130.36) (width 0.25) (layer "B.Cu") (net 27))
 (segment (start 156.21 96.52) (end 156.21 123.825) (width 1.27) (layer "F.Cu") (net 17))
 (segment (start 156.21 123.825) (end 147.955 132.08) (width 1.27) (layer "F.Cu") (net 17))
 (segment (start 163.168 93.699) (end 159.031 93.699) (width 1.27) (layer "F.Cu") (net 17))
 (segment (start 159.031 93.699) (end 156.21 96.52) (width 1.27) (layer "F.Cu") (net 17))
 (segment (start 147.955 132.08) (end 144.78 132.08) (width 1.27) (layer "F.Cu") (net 17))
 (segment (start 146.05 132.08) (end 144.78 132.08) (width 1.27) (layer "B.Cu") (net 17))
 (segment (start 155.04 141.07) (end 146.05 132.08) (width 1.27) (layer "B.Cu") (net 17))
 (segment (start 159.412 141.07) (end 155.04 141.07) (width 1.27) (layer "B.Cu") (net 17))
 (segment (start 142.24 100.33) (end 142.24 109.22) (width 0.25) (layer "F.Cu") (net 24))
 (segment (start 142.24 109.22) (end 144.78 111.76) (width 0.25) (layer "F.Cu") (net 24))
 (via (at 142.24 100.33) (size 0.8) (drill 0.4) (layers "F.Cu" "B.Cu") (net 24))
 (segment (start 163.168 101.319) (end 162.179 100.33) (width 0.25) (layer "B.Cu") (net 24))
 (segment (start 162.179 100.33) (end 142.24 100.33) (width 0.25) (layer "B.Cu") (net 24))
 (segment (start 163.168 103.859) (end 160.347 106.68) (width 0.25) (layer "B.Cu") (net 26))
 (segment (start 160.347 106.68) (end 144.78 106.68) (width 0.25) (layer "B.Cu") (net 26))
 (segment (start 163.168 106.399) (end 160.347 109.22) (width 0.25) (layer "B.Cu") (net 25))
 (segment (start 160.347 109.22) (end 144.78 109.22) (width 0.25) (layer "B.Cu") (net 25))
 (segment (start 127 101.6) (end 123.8758 101.6) (width 0.25) (layer "B.Cu") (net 7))
 (segment (start 161.617 110.49) (end 135.89 110.49) (width 0.25) (layer "B.Cu") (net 7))
 (segment (start 135.89 110.49) (end 127 101.6) (width 0.25) (layer "B.Cu") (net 7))
 (segment (start 163.168 108.939) (end 161.617 110.49) (width 0.25) (layer "B.Cu") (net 7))
 (segment (start 163.168 111.479) (end 161.617 113.03) (width 0.25) (layer "B.Cu") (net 8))
 (segment (start 161.617 113.03) (end 135.89 113.03) (width 0.25) (layer "B.Cu") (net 8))
 (segment (start 127 104.14) (end 123.8758 104.14) (width 0.25) (layer "B.Cu") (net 8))
 (segment (start 135.89 113.03) (end 127 104.14) (width 0.25) (layer "B.Cu") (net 8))
 (segment (start 97.2931 121.4485) (end 98.5885 121.4485) (width 0.25) (layer "B.Cu") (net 6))
 (segment (start 98.5885 121.4485) (end 104.14 127) (width 0.25) (layer "B.Cu") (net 6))
 (segment (start 139.7 127) (end 144.461802 122.238198) (width 0.25) (layer "B.Cu") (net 6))
 (segment (start 104.14 127) (end 139.7 127) (width 0.25) (layer "B.Cu") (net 6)))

